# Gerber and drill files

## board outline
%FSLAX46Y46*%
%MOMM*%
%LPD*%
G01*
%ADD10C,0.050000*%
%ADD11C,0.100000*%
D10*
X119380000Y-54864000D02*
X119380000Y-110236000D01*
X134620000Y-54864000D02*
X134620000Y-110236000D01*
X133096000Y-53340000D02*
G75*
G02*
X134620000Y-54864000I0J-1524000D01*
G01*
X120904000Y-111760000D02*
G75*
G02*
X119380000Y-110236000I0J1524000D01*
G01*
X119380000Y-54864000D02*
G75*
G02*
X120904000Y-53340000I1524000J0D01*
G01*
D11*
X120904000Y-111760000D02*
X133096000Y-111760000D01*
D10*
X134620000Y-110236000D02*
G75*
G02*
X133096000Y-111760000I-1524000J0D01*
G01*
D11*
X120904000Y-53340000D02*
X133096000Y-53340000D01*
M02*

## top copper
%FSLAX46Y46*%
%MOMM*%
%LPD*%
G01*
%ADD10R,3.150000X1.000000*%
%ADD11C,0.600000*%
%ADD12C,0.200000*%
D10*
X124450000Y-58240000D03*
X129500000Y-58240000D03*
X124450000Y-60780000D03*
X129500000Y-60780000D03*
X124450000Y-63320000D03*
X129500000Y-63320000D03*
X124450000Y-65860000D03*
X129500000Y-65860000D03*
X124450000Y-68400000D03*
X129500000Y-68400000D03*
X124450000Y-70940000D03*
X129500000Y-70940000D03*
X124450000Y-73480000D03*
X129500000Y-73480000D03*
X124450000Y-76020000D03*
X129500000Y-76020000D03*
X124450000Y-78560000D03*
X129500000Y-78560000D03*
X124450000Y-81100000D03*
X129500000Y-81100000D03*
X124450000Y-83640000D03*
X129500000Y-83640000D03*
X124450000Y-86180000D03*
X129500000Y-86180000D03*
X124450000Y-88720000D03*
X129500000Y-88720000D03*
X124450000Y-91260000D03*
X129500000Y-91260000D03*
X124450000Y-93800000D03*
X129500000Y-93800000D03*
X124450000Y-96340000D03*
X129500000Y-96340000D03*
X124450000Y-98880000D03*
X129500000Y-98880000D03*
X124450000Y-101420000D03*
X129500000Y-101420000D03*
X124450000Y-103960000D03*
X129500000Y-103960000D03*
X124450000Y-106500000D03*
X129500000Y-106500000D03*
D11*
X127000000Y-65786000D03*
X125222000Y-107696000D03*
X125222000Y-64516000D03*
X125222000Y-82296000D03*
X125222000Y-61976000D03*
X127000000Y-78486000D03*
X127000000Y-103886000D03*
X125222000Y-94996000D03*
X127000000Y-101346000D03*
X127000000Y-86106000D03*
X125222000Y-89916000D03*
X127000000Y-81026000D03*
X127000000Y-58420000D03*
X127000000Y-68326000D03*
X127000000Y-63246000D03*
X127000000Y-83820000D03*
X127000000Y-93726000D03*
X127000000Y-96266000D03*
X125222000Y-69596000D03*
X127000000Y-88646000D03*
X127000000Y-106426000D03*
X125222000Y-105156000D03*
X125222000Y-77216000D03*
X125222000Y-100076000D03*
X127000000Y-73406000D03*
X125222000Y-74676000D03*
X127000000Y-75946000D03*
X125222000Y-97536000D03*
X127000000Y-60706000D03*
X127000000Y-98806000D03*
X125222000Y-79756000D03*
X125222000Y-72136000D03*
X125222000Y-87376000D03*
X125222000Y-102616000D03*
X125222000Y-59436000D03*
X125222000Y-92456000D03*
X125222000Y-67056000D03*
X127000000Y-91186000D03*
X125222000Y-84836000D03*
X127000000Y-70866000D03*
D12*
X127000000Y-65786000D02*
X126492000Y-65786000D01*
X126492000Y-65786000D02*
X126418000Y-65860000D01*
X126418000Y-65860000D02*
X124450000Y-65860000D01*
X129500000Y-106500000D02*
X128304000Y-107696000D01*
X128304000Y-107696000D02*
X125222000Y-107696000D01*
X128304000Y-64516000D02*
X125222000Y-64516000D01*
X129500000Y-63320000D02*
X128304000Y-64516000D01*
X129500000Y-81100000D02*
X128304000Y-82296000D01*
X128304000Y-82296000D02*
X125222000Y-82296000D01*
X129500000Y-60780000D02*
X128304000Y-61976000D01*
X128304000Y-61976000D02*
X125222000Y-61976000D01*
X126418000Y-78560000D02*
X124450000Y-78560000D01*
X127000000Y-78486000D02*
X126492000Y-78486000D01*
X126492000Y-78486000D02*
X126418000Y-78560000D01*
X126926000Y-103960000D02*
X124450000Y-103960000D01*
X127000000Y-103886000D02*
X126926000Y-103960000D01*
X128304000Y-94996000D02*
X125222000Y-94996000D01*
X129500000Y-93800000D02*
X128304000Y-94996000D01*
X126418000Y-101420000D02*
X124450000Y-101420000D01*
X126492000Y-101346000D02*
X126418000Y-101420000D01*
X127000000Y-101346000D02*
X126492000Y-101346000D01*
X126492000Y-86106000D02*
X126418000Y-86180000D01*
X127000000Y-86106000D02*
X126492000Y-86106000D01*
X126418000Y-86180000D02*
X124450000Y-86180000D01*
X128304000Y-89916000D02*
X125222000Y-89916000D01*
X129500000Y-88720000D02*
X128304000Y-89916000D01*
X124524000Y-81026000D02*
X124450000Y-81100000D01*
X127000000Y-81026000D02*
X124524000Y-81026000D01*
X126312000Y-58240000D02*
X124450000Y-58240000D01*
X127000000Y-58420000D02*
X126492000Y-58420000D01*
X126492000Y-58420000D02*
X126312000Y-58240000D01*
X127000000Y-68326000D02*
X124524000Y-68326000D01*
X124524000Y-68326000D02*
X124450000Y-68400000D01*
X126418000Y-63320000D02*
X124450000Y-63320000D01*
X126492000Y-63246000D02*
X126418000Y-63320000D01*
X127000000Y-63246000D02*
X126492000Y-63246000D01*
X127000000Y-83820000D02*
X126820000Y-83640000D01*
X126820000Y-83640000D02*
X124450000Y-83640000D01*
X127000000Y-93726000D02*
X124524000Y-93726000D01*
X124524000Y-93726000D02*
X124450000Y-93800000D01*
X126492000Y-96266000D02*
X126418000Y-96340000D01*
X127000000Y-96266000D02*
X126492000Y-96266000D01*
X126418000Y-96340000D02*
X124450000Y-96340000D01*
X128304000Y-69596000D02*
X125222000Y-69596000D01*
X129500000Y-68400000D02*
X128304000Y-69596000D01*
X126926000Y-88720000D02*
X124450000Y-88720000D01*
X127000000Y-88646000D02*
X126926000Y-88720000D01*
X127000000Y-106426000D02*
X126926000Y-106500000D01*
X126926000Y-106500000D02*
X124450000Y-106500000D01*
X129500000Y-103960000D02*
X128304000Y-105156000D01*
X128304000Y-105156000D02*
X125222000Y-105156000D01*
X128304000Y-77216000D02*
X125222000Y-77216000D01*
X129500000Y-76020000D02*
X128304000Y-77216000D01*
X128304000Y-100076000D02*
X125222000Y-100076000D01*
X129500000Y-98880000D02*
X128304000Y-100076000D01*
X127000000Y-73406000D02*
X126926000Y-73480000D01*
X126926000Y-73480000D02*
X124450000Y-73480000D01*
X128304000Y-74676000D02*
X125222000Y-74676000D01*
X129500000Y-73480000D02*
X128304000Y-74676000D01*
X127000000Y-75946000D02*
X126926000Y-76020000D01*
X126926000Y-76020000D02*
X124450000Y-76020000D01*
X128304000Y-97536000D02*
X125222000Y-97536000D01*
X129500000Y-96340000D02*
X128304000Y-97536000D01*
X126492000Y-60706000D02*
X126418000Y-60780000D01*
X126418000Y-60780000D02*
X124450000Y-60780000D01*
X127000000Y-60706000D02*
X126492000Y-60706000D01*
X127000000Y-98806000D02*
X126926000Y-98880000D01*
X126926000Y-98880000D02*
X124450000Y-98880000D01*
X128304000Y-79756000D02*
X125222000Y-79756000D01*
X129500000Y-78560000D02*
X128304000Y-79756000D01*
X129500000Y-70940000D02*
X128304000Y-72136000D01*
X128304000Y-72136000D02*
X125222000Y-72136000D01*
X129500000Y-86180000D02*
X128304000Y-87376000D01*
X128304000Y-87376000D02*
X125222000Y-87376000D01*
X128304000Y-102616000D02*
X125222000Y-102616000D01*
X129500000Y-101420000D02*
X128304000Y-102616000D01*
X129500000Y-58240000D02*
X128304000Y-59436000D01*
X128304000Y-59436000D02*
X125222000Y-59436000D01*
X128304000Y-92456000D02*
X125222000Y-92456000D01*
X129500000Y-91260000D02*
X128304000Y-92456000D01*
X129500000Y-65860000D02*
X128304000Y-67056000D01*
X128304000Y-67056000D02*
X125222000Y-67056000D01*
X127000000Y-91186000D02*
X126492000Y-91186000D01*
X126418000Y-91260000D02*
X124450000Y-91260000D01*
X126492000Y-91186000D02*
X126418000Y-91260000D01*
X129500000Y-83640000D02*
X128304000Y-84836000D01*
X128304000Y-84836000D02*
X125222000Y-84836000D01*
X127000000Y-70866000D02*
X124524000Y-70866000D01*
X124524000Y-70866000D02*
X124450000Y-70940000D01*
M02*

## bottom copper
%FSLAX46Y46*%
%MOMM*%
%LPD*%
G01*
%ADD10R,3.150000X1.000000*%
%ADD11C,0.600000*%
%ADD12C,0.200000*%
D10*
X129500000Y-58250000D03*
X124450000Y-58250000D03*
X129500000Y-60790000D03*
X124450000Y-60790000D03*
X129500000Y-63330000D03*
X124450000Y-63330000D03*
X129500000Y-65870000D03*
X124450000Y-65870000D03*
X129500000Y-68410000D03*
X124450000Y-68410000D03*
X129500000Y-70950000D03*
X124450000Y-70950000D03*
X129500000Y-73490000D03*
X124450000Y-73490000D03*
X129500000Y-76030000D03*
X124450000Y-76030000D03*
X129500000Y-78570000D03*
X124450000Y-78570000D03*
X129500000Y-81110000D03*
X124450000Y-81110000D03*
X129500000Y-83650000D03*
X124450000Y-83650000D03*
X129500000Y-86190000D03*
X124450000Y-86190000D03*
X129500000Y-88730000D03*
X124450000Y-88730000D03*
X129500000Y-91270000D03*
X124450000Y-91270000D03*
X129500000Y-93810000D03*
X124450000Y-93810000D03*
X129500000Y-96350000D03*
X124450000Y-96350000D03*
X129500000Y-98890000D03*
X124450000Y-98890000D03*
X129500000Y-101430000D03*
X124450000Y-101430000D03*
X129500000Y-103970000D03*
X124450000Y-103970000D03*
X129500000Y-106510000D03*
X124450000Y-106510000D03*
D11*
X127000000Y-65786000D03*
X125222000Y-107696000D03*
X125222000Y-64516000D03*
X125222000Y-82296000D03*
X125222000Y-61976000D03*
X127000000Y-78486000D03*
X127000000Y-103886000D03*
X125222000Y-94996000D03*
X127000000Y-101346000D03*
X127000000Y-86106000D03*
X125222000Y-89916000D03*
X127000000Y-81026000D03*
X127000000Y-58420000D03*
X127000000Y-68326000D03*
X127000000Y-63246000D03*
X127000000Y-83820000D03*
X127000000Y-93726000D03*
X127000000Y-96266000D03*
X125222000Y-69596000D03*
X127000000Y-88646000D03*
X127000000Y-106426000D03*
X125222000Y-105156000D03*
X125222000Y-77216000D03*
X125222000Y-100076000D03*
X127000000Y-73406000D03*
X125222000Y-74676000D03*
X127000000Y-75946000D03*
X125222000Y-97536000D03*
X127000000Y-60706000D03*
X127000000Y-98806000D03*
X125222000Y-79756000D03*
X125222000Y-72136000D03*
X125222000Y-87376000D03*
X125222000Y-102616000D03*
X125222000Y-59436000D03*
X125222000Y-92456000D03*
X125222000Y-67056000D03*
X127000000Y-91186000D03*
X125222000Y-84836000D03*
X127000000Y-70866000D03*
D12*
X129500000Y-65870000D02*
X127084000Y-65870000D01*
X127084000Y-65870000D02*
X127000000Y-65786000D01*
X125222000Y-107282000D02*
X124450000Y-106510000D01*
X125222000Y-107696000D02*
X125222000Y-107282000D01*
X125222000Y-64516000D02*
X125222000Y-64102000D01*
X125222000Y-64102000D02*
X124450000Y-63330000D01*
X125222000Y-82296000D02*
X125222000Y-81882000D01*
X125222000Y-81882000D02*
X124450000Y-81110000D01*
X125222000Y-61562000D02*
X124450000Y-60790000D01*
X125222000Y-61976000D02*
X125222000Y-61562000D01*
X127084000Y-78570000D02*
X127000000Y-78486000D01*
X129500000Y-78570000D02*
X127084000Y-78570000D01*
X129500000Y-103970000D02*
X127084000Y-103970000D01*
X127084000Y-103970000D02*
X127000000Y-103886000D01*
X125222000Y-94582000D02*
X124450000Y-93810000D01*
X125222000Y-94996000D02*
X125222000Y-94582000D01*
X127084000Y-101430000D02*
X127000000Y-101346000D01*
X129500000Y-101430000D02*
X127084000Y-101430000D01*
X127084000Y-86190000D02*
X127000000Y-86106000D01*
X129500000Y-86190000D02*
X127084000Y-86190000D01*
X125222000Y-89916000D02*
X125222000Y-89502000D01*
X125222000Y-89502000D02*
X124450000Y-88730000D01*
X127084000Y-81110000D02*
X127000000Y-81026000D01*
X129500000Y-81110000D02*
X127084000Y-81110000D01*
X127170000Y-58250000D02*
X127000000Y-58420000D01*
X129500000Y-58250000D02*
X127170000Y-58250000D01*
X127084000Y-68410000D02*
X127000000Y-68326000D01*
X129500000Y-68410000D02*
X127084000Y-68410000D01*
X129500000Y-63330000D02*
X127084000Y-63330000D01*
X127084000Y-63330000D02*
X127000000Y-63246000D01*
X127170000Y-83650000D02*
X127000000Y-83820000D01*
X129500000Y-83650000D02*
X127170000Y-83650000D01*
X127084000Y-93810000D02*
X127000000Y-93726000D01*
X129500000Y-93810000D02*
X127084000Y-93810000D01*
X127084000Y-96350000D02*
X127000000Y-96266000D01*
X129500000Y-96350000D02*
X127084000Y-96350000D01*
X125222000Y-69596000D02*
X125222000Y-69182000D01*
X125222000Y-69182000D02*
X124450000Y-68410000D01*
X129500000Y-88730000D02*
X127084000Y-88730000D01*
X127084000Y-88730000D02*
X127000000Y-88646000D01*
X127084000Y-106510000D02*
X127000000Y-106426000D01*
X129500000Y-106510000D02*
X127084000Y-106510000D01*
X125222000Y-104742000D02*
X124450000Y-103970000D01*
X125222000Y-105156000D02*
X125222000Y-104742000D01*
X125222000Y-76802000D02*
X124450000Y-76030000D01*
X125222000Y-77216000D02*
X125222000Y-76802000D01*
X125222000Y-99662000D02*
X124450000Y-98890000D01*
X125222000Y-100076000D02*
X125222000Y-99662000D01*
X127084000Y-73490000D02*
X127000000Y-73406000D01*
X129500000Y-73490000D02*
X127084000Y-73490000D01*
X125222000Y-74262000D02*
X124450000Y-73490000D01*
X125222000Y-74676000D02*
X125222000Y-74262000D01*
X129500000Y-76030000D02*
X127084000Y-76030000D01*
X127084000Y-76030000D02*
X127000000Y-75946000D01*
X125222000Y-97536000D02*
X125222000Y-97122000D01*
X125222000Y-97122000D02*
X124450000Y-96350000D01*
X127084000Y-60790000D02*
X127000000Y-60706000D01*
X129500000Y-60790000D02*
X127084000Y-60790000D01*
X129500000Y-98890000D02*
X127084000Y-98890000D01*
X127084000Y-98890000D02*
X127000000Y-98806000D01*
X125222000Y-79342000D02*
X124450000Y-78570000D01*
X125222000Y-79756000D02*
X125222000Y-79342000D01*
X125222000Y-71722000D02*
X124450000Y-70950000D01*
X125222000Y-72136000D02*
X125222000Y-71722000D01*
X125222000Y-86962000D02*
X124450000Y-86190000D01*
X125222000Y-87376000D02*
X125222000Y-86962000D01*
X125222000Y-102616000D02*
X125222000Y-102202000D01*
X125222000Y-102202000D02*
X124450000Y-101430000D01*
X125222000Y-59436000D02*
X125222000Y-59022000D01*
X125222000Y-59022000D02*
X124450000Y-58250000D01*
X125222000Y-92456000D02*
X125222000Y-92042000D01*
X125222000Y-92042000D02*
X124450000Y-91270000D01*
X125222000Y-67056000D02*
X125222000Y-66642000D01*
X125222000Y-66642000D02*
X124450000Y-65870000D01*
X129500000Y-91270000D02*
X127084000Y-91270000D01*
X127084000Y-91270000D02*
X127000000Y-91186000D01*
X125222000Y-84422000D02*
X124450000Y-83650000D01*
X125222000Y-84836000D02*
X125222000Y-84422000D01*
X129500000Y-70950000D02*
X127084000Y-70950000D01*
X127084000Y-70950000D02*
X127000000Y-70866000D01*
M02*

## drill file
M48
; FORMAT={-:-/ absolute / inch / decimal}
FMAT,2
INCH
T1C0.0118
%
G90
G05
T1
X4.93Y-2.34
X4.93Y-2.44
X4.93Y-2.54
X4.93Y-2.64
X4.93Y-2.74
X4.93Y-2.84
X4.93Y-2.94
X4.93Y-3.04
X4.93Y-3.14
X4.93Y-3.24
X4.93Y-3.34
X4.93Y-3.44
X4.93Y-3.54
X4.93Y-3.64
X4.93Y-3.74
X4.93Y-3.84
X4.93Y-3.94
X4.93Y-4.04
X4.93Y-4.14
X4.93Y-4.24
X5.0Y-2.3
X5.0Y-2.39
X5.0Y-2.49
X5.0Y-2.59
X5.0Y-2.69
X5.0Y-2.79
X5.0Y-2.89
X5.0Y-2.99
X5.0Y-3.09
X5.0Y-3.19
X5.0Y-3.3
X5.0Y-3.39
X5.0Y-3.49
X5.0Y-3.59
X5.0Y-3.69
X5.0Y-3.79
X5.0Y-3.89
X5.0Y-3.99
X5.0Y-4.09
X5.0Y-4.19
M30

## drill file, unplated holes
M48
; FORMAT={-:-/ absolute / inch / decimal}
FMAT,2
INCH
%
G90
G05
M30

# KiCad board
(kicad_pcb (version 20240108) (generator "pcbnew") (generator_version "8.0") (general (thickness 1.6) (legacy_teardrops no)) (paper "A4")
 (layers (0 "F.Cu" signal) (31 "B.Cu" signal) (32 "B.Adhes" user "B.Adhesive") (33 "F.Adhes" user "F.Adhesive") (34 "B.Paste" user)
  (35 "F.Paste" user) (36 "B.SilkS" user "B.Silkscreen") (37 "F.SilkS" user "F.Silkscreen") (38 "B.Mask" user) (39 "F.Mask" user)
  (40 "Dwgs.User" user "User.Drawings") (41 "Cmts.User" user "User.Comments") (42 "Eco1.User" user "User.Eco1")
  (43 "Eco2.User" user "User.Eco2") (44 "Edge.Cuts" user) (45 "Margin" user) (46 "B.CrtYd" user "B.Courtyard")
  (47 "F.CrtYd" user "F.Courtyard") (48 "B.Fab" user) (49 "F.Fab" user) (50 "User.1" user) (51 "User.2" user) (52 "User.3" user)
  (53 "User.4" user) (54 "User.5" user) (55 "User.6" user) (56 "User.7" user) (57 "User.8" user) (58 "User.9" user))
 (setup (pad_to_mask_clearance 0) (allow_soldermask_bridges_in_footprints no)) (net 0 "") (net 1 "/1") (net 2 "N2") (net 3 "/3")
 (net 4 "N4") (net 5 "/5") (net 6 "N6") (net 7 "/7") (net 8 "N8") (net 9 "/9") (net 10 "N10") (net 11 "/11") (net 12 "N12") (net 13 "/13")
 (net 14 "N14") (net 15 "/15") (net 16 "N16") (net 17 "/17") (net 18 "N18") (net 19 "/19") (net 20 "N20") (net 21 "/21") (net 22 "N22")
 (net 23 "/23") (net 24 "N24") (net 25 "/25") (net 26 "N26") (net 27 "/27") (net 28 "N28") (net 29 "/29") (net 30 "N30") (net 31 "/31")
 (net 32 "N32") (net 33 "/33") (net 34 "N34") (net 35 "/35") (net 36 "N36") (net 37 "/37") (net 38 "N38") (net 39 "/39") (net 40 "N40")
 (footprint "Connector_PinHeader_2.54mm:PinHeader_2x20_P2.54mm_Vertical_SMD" (layer "F.Cu") (at 126.975 82.37)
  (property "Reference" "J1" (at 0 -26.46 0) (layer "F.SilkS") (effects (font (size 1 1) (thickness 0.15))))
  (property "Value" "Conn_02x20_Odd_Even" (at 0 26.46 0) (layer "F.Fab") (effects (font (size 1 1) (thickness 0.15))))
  (pad "1" smd rect (at -2.525 -24.13) (size 3.15 1) (layers "F.Cu" "F.Paste" "F.Mask") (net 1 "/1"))
  (pad "2" smd rect (at 2.525 -24.13) (size 3.15 1) (layers "F.Cu" "F.Paste" "F.Mask") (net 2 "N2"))
  (pad "3" smd rect (at -2.525 -21.59) (size 3.15 1) (layers "F.Cu" "F.Paste" "F.Mask") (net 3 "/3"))
  (pad "4" smd rect (at 2.525 -21.59) (size 3.15 1) (layers "F.Cu" "F.Paste" "F.Mask") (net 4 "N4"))
  (pad "5" smd rect (at -2.525 -19.05) (size 3.15 1) (layers "F.Cu" "F.Paste" "F.Mask") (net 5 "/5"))
  (pad "6" smd rect (at 2.525 -19.05) (size 3.15 1) (layers "F.Cu" "F.Paste" "F.Mask") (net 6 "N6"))
  (pad "7" smd rect (at -2.525 -16.51) (size 3.15 1) (layers "F.Cu" "F.Paste" "F.Mask") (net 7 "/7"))
  (pad "8" smd rect (at 2.525 -16.51) (size 3.15 1) (layers "F.Cu" "F.Paste" "F.Mask") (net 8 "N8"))
  (pad "9" smd rect (at -2.525 -13.97) (size 3.15 1) (layers "F.Cu" "F.Paste" "F.Mask") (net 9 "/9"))
  (pad "10" smd rect (at 2.525 -13.97) (size 3.15 1) (layers "F.Cu" "F.Paste" "F.Mask") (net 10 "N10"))
  (pad "11" smd rect (at -2.525 -11.43) (size 3.15 1) (layers "F.Cu" "F.Paste" "F.Mask") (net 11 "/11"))
  (pad "12" smd rect (at 2.525 -11.43) (size 3.15 1) (layers "F.Cu" "F.Paste" "F.Mask") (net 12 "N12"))
  (pad "13" smd rect (at -2.525 -8.89) (size 3.15 1) (layers "F.Cu" "F.Paste" "F.Mask") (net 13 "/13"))
  (pad "14" smd rect (at 2.525 -8.89) (size 3.15 1) (layers "F.Cu" "F.Paste" "F.Mask") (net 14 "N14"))
  (pad "15" smd rect (at -2.525 -6.35) (size 3.15 1) (layers "F.Cu" "F.Paste" "F.Mask") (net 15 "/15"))
  (pad "16" smd rect (at 2.525 -6.35) (size 3.15 1) (layers "F.Cu" "F.Paste" "F.Mask") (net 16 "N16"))
  (pad "17" smd rect (at -2.525 -3.81) (size 3.15 1) (layers "F.Cu" "F.Paste" "F.Mask") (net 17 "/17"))
  (pad "18" smd rect (at 2.525 -3.81) (size 3.15 1) (layers "F.Cu" "F.Paste" "F.Mask") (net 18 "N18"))
  (pad "19" smd rect (at -2.525 -1.27) (size 3.15 1) (layers "F.Cu" "F.Paste" "F.Mask") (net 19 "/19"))
  (pad "20" smd rect (at 2.525 -1.27) (size 3.15 1) (layers "F.Cu" "F.Paste" "F.Mask") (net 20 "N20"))
  (pad "21" smd rect (at -2.525 1.27) (size 3.15 1) (layers "F.Cu" "F.Paste" "F.Mask") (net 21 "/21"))
  (pad "22" smd rect (at 2.525 1.27) (size 3.15 1) (layers "F.Cu" "F.Paste" "F.Mask") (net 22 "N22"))
  (pad "23" smd rect (at -2.525 3.81) (size 3.15 1) (layers "F.Cu" "F.Paste" "F.Mask") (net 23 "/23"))
  (pad "24" smd rect (at 2.525 3.81) (size 3.15 1) (layers "F.Cu" "F.Paste" "F.Mask") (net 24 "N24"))
  (pad "25" smd rect (at -2.525 6.35) (size 3.15 1) (layers "F.Cu" "F.Paste" "F.Mask") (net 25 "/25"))
  (pad "26" smd rect (at 2.525 6.35) (size 3.15 1) (layers "F.Cu" "F.Paste" "F.Mask") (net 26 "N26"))
  (pad "27" smd rect (at -2.525 8.89) (size 3.15 1) (layers "F.Cu" "F.Paste" "F.Mask") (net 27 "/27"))
  (pad "28" smd rect (at 2.525 8.89) (size 3.15 1) (layers "F.Cu" "F.Paste" "F.Mask") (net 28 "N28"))
  (pad "29" smd rect (at -2.525 11.43) (size 3.15 1) (layers "F.Cu" "F.Paste" "F.Mask") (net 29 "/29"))
  (pad "30" smd rect (at 2.525 11.43) (size 3.15 1) (layers "F.Cu" "F.Paste" "F.Mask") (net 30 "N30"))
  (pad "31" smd rect (at -2.525 13.97) (size 3.15 1) (layers "F.Cu" "F.Paste" "F.Mask") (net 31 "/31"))
  (pad "32" smd rect (at 2.525 13.97) (size 3.15 1) (layers "F.Cu" "F.Paste" "F.Mask") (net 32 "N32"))
  (pad "33" smd rect (at -2.525 16.51) (size 3.15 1) (layers "F.Cu" "F.Paste" "F.Mask") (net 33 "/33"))
  (pad "34" smd rect (at 2.525 16.51) (size 3.15 1) (layers "F.Cu" "F.Paste" "F.Mask") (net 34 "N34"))
  (pad "35" smd rect (at -2.525 19.05) (size 3.15 1) (layers "F.Cu" "F.Paste" "F.Mask") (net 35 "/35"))
  (pad "36" smd rect (at 2.525 19.05) (size 3.15 1) (layers "F.Cu" "F.Paste" "F.Mask") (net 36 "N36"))
  (pad "37" smd rect (at -2.525 21.59) (size 3.15 1) (layers "F.Cu" "F.Paste" "F.Mask") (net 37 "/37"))
  (pad "38" smd rect (at 2.525 21.59) (size 3.15 1) (layers "F.Cu" "F.Paste" "F.Mask") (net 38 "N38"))
  (pad "39" smd rect (at -2.525 24.13) (size 3.15 1) (layers "F.Cu" "F.Paste" "F.Mask") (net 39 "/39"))
  (pad "40" smd rect (at 2.525 24.13) (size 3.15 1) (layers "F.Cu" "F.Paste" "F.Mask") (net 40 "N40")))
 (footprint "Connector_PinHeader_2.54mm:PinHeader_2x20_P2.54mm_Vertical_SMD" (layer "B.Cu") (at 126.975 82.38 180)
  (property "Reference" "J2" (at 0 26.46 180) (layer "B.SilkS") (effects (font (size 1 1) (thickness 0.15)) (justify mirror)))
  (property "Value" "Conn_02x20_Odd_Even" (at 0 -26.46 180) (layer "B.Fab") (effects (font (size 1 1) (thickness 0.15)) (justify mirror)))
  (pad "1" smd rect (at -2.525 24.13 180) (size 3.15 1) (layers "B.Cu" "B.Paste" "B.Mask") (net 1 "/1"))
  (pad "2" smd rect (at 2.525 24.13 180) (size 3.15 1) (layers "B.Cu" "B.Paste" "B.Mask") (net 2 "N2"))
  (pad "3" smd rect (at -2.525 21.59 180) (size 3.15 1) (layers "B.Cu" "B.Paste" "B.Mask") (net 3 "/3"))
  (pad "4" smd rect (at 2.525 21.59 180) (size 3.15 1) (layers "B.Cu" "B.Paste" "B.Mask") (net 4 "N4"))
  (pad "5" smd rect (at -2.525 19.05 180) (size 3.15 1) (layers "B.Cu" "B.Paste" "B.Mask") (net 5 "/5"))
  (pad "6" smd rect (at 2.525 19.05 180) (size 3.15 1) (layers "B.Cu" "B.Paste" "B.Mask") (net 6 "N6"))
  (pad "7" smd rect (at -2.525 16.51 180) (size 3.15 1) (layers "B.Cu" "B.Paste" "B.Mask") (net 7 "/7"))
  (pad "8" smd rect (at 2.525 16.51 180) (size 3.15 1) (layers "B.Cu" "B.Paste" "B.Mask") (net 8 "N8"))
  (pad "9" smd rect (at -2.525 13.97 180) (size 3.15 1) (layers "B.Cu" "B.Paste" "B.Mask") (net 9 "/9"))
  (pad "10" smd rect (at 2.525 13.97 180) (size 3.15 1) (layers "B.Cu" "B.Paste" "B.Mask") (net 10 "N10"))
  (pad "11" smd rect (at -2.525 11.43 180) (size 3.15 1) (layers "B.Cu" "B.Paste" "B.Mask") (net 11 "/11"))
  (pad "12" smd rect (at 2.525 11.43 180) (size 3.15 1) (layers "B.Cu" "B.Paste" "B.Mask") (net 12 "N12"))
  (pad "13" smd rect (at -2.525 8.89 180) (size 3.15 1) (layers "B.Cu" "B.Paste" "B.Mask") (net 13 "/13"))
  (pad "14" smd rect (at 2.525 8.89 180) (size 3.15 1) (layers "B.Cu" "B.Paste" "B.Mask") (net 14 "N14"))
  (pad "15" smd rect (at -2.525 6.35 180) (size 3.15 1) (layers "B.Cu" "B.Paste" "B.Mask") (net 15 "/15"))
  (pad "16" smd rect (at 2.525 6.35 180) (size 3.15 1) (layers "B.Cu" "B.Paste" "B.Mask") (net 16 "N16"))
  (pad "17" smd rect (at -2.525 3.81 180) (size 3.15 1) (layers "B.Cu" "B.Paste" "B.Mask") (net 17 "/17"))
  (pad "18" smd rect (at 2.525 3.81 180) (size 3.15 1) (layers "B.Cu" "B.Paste" "B.Mask") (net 18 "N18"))
  (pad "19" smd rect (at -2.525 1.27 180) (size 3.15 1) (layers "B.Cu" "B.Paste" "B.Mask") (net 19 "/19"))
  (pad "20" smd rect (at 2.525 1.27 180) (size 3.15 1) (layers "B.Cu" "B.Paste" "B.Mask") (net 20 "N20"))
  (pad "21" smd rect (at -2.525 -1.27 180) (size 3.15 1) (layers "B.Cu" "B.Paste" "B.Mask") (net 21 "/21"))
  (pad "22" smd rect (at 2.525 -1.27 180) (size 3.15 1) (layers "B.Cu" "B.Paste" "B.Mask") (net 22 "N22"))
  (pad "23" smd rect (at -2.525 -3.81 180) (size 3.15 1) (layers "B.Cu" "B.Paste" "B.Mask") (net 23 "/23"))
  (pad "24" smd rect (at 2.525 -3.81 180) (size 3.15 1) (layers "B.Cu" "B.Paste" "B.Mask") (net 24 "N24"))
  (pad "25" smd rect (at -2.525 -6.35 180) (size 3.15 1) (layers "B.Cu" "B.Paste" "B.Mask") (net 25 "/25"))
  (pad "26" smd rect (at 2.525 -6.35 180) (size 3.15 1) (layers "B.Cu" "B.Paste" "B.Mask") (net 26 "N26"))
  (pad "27" smd rect (at -2.525 -8.89 180) (size 3.15 1) (layers "B.Cu" "B.Paste" "B.Mask") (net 27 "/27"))
  (pad "28" smd rect (at 2.525 -8.89 180) (size 3.15 1) (layers "B.Cu" "B.Paste" "B.Mask") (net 28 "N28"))
  (pad "29" smd rect (at -2.525 -11.43 180) (size 3.15 1) (layers "B.Cu" "B.Paste" "B.Mask") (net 29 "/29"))
  (pad "30" smd rect (at 2.525 -11.43 180) (size 3.15 1) (layers "B.Cu" "B.Paste" "B.Mask") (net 30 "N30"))
  (pad "31" smd rect (at -2.525 -13.97 180) (size 3.15 1) (layers "B.Cu" "B.Paste" "B.Mask") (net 31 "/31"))
  (pad "32" smd rect (at 2.525 -13.97 180) (size 3.15 1) (layers "B.Cu" "B.Paste" "B.Mask") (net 32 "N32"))
  (pad "33" smd rect (at -2.525 -16.51 180) (size 3.15 1) (layers "B.Cu" "B.Paste" "B.Mask") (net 33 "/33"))
  (pad "34" smd rect (at 2.525 -16.51 180) (size 3.15 1) (layers "B.Cu" "B.Paste" "B.Mask") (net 34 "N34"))
  (pad "35" smd rect (at -2.525 -19.05 180) (size 3.15 1) (layers "B.Cu" "B.Paste" "B.Mask") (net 35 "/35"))
  (pad "36" smd rect (at 2.525 -19.05 180) (size 3.15 1) (layers "B.Cu" "B.Paste" "B.Mask") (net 36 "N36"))
  (pad "37" smd rect (at -2.525 -21.59 180) (size 3.15 1) (layers "B.Cu" "B.Paste" "B.Mask") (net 37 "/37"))
  (pad "38" smd rect (at 2.525 -21.59 180) (size 3.15 1) (layers "B.Cu" "B.Paste" "B.Mask") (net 38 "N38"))
  (pad "39" smd rect (at -2.525 -24.13 180) (size 3.15 1) (layers "B.Cu" "B.Paste" "B.Mask") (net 39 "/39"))
  (pad "40" smd rect (at 2.525 -24.13 180) (size 3.15 1) (layers "B.Cu" "B.Paste" "B.Mask") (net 40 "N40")))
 (gr_line (start 119.38 54.864) (end 119.38 110.236) (stroke (width 0.05) (type default)) (layer "Edge.Cuts"))
 (gr_line (start 134.62 54.864) (end 134.62 110.236) (stroke (width 0.05) (type default)) (layer "Edge.Cuts"))
 (gr_arc (start 133.096 53.34) (mid 134.173631 53.786369) (end 134.62 54.864) (stroke (width 0.05) (type default)) (layer "Edge.Cuts"))
 (gr_arc (start 120.904 111.76) (mid 119.826369 111.313631) (end 119.38 110.236) (stroke (width 0.05) (type default)) (layer "Edge.Cuts"))
 (gr_arc (start 119.38 54.864) (mid 119.826369 53.786369) (end 120.904 53.34) (stroke (width 0.05) (type default)) (layer "Edge.Cuts"))
 (gr_line (start 120.904 111.76) (end 133.096 111.76) (stroke (width 0.1) (type default)) (layer "Edge.Cuts"))
 (gr_arc (start 134.62 110.236) (mid 134.173631 111.313631) (end 133.096 111.76) (stroke (width 0.05) (type default)) (layer "Edge.Cuts"))
 (gr_line (start 120.904 53.34) (end 133.096 53.34) (stroke (width 0.1) (type default)) (layer "Edge.Cuts"))
 (segment (start 127 65.786) (end 126.492 65.786) (width 0.2) (layer "F.Cu") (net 7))
 (segment (start 126.492 65.786) (end 126.418 65.86) (width 0.2) (layer "F.Cu") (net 7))
 (segment (start 126.418 65.86) (end 124.45 65.86) (width 0.2) (layer "F.Cu") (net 7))
 (via (at 127 65.786) (size 0.6) (drill 0.3) (layers "F.Cu" "B.Cu") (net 7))
 (segment (start 129.5 65.87) (end 127.084 65.87) (width 0.2) (layer "B.Cu") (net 7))
 (segment (start 127.084 65.87) (end 127 65.786) (width 0.2) (layer "B.Cu") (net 7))
 (segment (start 129.5 106.5) (end 128.304 107.696) (width 0.2) (layer "F.Cu") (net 40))
 (segment (start 128.304 107.696) (end 125.222 107.696) (width 0.2) (layer "F.Cu") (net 40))
 (via (at 125.222 107.696) (size 0.6) (drill 0.3) (layers "F.Cu" "B.Cu") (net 40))
 (segment (start 125.222 107.282) (end 124.45 106.51) (width 0.2) (layer "B.Cu") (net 40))
 (segment (start 125.222 107.696) (end 125.222 107.282) (width 0.2) (layer "B.Cu") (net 40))
 (segment (start 128.304 64.516) (end 125.222 64.516) (width 0.2) (layer "F.Cu") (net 6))
 (segment (start 129.5 63.32) (end 128.304 64.516) (width 0.2) (layer "F.Cu") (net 6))
 (via (at 125.222 64.516) (size 0.6) (drill 0.3) (layers "F.Cu" "B.Cu") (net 6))
 (segment (start 125.222 64.516) (end 125.222 64.102) (width 0.2) (layer "B.Cu") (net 6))
 (segment (start 125.222 64.102) (end 124.45 63.33) (width 0.2) (layer "B.Cu") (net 6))
 (segment (start 129.5 81.1) (end 128.304 82.296) (width 0.2) (layer "F.Cu") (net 20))
 (segment (start 128.304 82.296) (end 125.222 82.296) (width 0.2) (layer "F.Cu") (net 20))
 (via (at 125.222 82.296) (size 0.6) (drill 0.3) (layers "F.Cu" "B.Cu") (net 20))
 (segment (start 125.222 82.296) (end 125.222 81.882) (width 0.2) (layer "B.Cu") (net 20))
 (segment (start 125.222 81.882) (end 124.45 81.11) (width 0.2) (layer "B.Cu") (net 20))
 (segment (start 129.5 60.78) (end 128.304 61.976) (width 0.2) (layer "F.Cu") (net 4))
 (segment (start 128.304 61.976) (end 125.222 61.976) (width 0.2) (layer "F.Cu") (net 4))
 (via (at 125.222 61.976) (size 0.6) (drill 0.3) (layers "F.Cu" "B.Cu") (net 4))
 (segment (start 125.222 61.562) (end 124.45 60.79) (width 0.2) (layer "B.Cu") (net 4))
 (segment (start 125.222 61.976) (end 125.222 61.562) (width 0.2) (layer "B.Cu") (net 4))
 (segment (start 126.418 78.56) (end 124.45 78.56) (width 0.2) (layer "F.Cu") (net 17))
 (segment (start 127 78.486) (end 126.492 78.486) (width 0.2) (layer "F.Cu") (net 17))
 (segment (start 126.492 78.486) (end 126.418 78.56) (width 0.2) (layer "F.Cu") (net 17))
 (via (at 127 78.486) (size 0.6) (drill 0.3) (layers "F.Cu" "B.Cu") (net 17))
 (segment (start 127.084 78.57) (end 127 78.486) (width 0.2) (layer "B.Cu") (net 17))
 (segment (start 129.5 78.57) (end 127.084 78.57) (width 0.2) (layer "B.Cu") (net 17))
 (segment (start 126.926 103.96) (end 124.45 103.96) (width 0.2) (layer "F.Cu") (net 37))
 (segment (start 127 103.886) (end 126.926 103.96) (width 0.2) (layer "F.Cu") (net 37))
 (via (at 127 103.886) (size 0.6) (drill 0.3) (layers "F.Cu" "B.Cu") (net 37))
 (segment (start 129.5 103.97) (end 127.084 103.97) (width 0.2) (layer "B.Cu") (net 37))
 (segment (start 127.084 103.97) (end 127 103.886) (width 0.2) (layer "B.Cu") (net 37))
 (segment (start 128.304 94.996) (end 125.222 94.996) (width 0.2) (layer "F.Cu") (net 30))
 (segment (start 129.5 93.8) (end 128.304 94.996) (width 0.2) (layer "F.Cu") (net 30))
 (via (at 125.222 94.996) (size 0.6) (drill 0.3) (layers "F.Cu" "B.Cu") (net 30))
 (segment (start 125.222 94.582) (end 124.45 93.81) (width 0.2) (layer "B.Cu") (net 30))
 (segment (start 125.222 94.996) (end 125.222 94.582) (width 0.2) (layer "B.Cu") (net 30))
 (segment (start 126.418 101.42) (end 124.45 101.42) (width 0.2) (layer "F.Cu") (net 35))
 (segment (start 126.492 101.346) (end 126.418 101.42) (width 0.2) (layer "F.Cu") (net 35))
 (segment (start 127 101.346) (end 126.492 101.346) (width 0.2) (layer "F.Cu") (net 35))
 (via (at 127 101.346) (size 0.6) (drill 0.3) (layers "F.Cu" "B.Cu") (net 35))
 (segment (start 127.084 101.43) (end 127 101.346) (width 0.2) (layer "B.Cu") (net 35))
 (segment (start 129.5 101.43) (end 127.084 101.43) (width 0.2) (layer "B.Cu") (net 35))
 (segment (start 126.492 86.106) (end 126.418 86.18) (width 0.2) (layer "F.Cu") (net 23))
 (segment (start 127 86.106) (end 126.492 86.106) (width 0.2) (layer "F.Cu") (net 23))
 (segment (start 126.418 86.18) (end 124.45 86.18) (width 0.2) (layer "F.Cu") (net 23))
 (via (at 127 86.106) (size 0.6) (drill 0.3) (layers "F.Cu" "B.Cu") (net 23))
 (segment (start 127.084 86.19) (end 127 86.106) (width 0.2) (layer "B.Cu") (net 23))
 (segment (start 129.5 86.19) (end 127.084 86.19) (width 0.2) (layer "B.Cu") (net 23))
 (segment (start 128.304 89.916) (end 125.222 89.916) (width 0.2) (layer "F.Cu") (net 26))
 (segment (start 129.5 88.72) (end 128.304 89.916) (width 0.2) (layer "F.Cu") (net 26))
 (via (at 125.222 89.916) (size 0.6) (drill 0.3) (layers "F.Cu" "B.Cu") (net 26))
 (segment (start 125.222 89.916) (end 125.222 89.502) (width 0.2) (layer "B.Cu") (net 26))
 (segment (start 125.222 89.502) (end 124.45 88.73) (width 0.2) (layer "B.Cu") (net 26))
 (segment (start 124.524 81.026) (end 124.45 81.1) (width 0.2) (layer "F.Cu") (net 19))
 (segment (start 127 81.026) (end 124.524 81.026) (width 0.2) (layer "F.Cu") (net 19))
 (via (at 127 81.026) (size 0.6) (drill 0.3) (layers "F.Cu" "B.Cu") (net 19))
 (segment (start 127.084 81.11) (end 127 81.026) (width 0.2) (layer "B.Cu") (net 19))
 (segment (start 129.5 81.11) (end 127.084 81.11) (width 0.2) (layer "B.Cu") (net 19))
 (segment (start 126.312 58.24) (end 124.45 58.24) (width 0.2) (layer "F.Cu") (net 1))
 (segment (start 127 58.42) (end 126.492 58.42) (width 0.2) (layer "F.Cu") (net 1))
 (segment (start 126.492 58.42) (end 126.312 58.24) (width 0.2) (layer "F.Cu") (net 1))
 (via (at 127 58.42) (size 0.6) (drill 0.3) (layers "F.Cu" "B.Cu") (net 1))
 (segment (start 127.17 58.25) (end 127 58.42) (width 0.2) (layer "B.Cu") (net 1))
 (segment (start 129.5 58.25) (end 127.17 58.25) (width 0.2) (layer "B.Cu") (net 1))
 (segment (start 127 68.326) (end 124.524 68.326) (width 0.2) (layer "F.Cu") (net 9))
 (segment (start 124.524 68.326) (end 124.45 68.4) (width 0.2) (layer "F.Cu") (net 9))
 (via (at 127 68.326) (size 0.6) (drill 0.3) (layers "F.Cu" "B.Cu") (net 9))
 (segment (start 127.084 68.41) (end 127 68.326) (width 0.2) (layer "B.Cu") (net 9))
 (segment (start 129.5 68.41) (end 127.084 68.41) (width 0.2) (layer "B.Cu") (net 9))
 (segment (start 126.418 63.32) (end 124.45 63.32) (width 0.2) (layer "F.Cu") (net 5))
 (segment (start 126.492 63.246) (end 126.418 63.32) (width 0.2) (layer "F.Cu") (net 5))
 (segment (start 127 63.246) (end 126.492 63.246) (width 0.2) (layer "F.Cu") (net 5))
 (via (at 127 63.246) (size 0.6) (drill 0.3) (layers "F.Cu" "B.Cu") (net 5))
 (segment (start 129.5 63.33) (end 127.084 63.33) (width 0.2) (layer "B.Cu") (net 5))
 (segment (start 127.084 63.33) (end 127 63.246) (width 0.2) (layer "B.Cu") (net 5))
 (segment (start 127 83.82) (end 126.82 83.64) (width 0.2) (layer "F.Cu") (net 21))
 (segment (start 126.82 83.64) (end 124.45 83.64) (width 0.2) (layer "F.Cu") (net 21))
 (via (at 127 83.82) (size 0.6) (drill 0.3) (layers "F.Cu" "B.Cu") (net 21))
 (segment (start 127.17 83.65) (end 127 83.82) (width 0.2) (layer "B.Cu") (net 21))
 (segment (start 129.5 83.65) (end 127.17 83.65) (width 0.2) (layer "B.Cu") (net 21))
 (segment (start 127 93.726) (end 124.524 93.726) (width 0.2) (layer "F.Cu") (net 29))
 (segment (start 124.524 93.726) (end 124.45 93.8) (width 0.2) (layer "F.Cu") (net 29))
 (via (at 127 93.726) (size 0.6) (drill 0.3) (layers "F.Cu" "B.Cu") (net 29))
 (segment (start 127.084 93.81) (end 127 93.726) (width 0.2) (layer "B.Cu") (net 29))
 (segment (start 129.5 93.81) (end 127.084 93.81) (width 0.2) (layer "B.Cu") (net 29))
 (segment (start 126.492 96.266) (end 126.418 96.34) (width 0.2) (layer "F.Cu") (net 31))
 (segment (start 127 96.266) (end 126.492 96.266) (width 0.2) (layer "F.Cu") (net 31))
 (segment (start 126.418 96.34) (end 124.45 96.34) (width 0.2) (layer "F.Cu") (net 31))
 (via (at 127 96.266) (size 0.6) (drill 0.3) (layers "F.Cu" "B.Cu") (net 31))
 (segment (start 127.084 96.35) (end 127 96.266) (width 0.2) (layer "B.Cu") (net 31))
 (segment (start 129.5 96.35) (end 127.084 96.35) (width 0.2) (layer "B.Cu") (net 31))
 (segment (start 128.304 69.596) (end 125.222 69.596) (width 0.2) (layer "F.Cu") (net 10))
 (segment (start 129.5 68.4) (end 128.304 69.596) (width 0.2) (layer "F.Cu") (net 10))
 (via (at 125.222 69.596) (size 0.6) (drill 0.3) (layers "F.Cu" "B.Cu") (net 10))
 (segment (start 125.222 69.596) (end 125.222 69.182) (width 0.2) (layer "B.Cu") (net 10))
 (segment (start 125.222 69.182) (end 124.45 68.41) (width 0.2) (layer "B.Cu") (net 10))
 (segment (start 126.926 88.72) (end 124.45 88.72) (width 0.2) (layer "F.Cu") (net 25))
 (segment (start 127 88.646) (end 126.926 88.72) (width 0.2) (layer "F.Cu") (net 25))
 (via (at 127 88.646) (size 0.6) (drill 0.3) (layers "F.Cu" "B.Cu") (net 25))
 (segment (start 129.5 88.73) (end 127.084 88.73) (width 0.2) (layer "B.Cu") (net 25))
 (segment (start 127.084 88.73) (end 127 88.646) (width 0.2) (layer "B.Cu") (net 25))
 (segment (start 127 106.426) (end 126.926 106.5) (width 0.2) (layer "F.Cu") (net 39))
 (segment (start 126.926 106.5) (end 124.45 106.5) (width 0.2) (layer "F.Cu") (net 39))
 (via (at 127 106.426) (size 0.6) (drill 0.3) (layers "F.Cu" "B.Cu") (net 39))
 (segment (start 127.084 106.51) (end 127 106.426) (width 0.2) (layer "B.Cu") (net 39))
 (segment (start 129.5 106.51) (end 127.084 106.51) (width 0.2) (layer "B.Cu") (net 39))
 (segment (start 129.5 103.96) (end 128.304 105.156) (width 0.2) (layer "F.Cu") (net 38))
 (segment (start 128.304 105.156) (end 125.222 105.156) (width 0.2) (layer "F.Cu") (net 38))
 (via (at 125.222 105.156) (size 0.6) (drill 0.3) (layers "F.Cu" "B.Cu") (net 38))
 (segment (start 125.222 104.742) (end 124.45 103.97) (width 0.2) (layer "B.Cu") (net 38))
 (segment (start 125.222 105.156) (end 125.222 104.742) (width 0.2) (layer "B.Cu") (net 38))
 (segment (start 128.304 77.216) (end 125.222 77.216) (width 0.2) (layer "F.Cu") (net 16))
 (segment (start 129.5 76.02) (end 128.304 77.216) (width 0.2) (layer "F.Cu") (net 16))
 (via (at 125.222 77.216) (size 0.6) (drill 0.3) (layers "F.Cu" "B.Cu") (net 16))
 (segment (start 125.222 76.802) (end 124.45 76.03) (width 0.2) (layer "B.Cu") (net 16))
 (segment (start 125.222 77.216) (end 125.222 76.802) (width 0.2) (layer "B.Cu") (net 16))
 (segment (start 128.304 100.076) (end 125.222 100.076) (width 0.2) (layer "F.Cu") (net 34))
 (segment (start 129.5 98.88) (end 128.304 100.076) (width 0.2) (layer "F.Cu") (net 34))
 (via (at 125.222 100.076) (size 0.6) (drill 0.3) (layers "F.Cu" "B.Cu") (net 34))
 (segment (start 125.222 99.662) (end 124.45 98.89) (width 0.2) (layer "B.Cu") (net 34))
 (segment (start 125.222 100.076) (end 125.222 99.662) (width 0.2) (layer "B.Cu") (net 34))
 (segment (start 127 73.406) (end 126.926 73.48) (width 0.2) (layer "F.Cu") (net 13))
 (segment (start 126.926 73.48) (end 124.45 73.48) (width 0.2) (layer "F.Cu") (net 13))
 (via (at 127 73.406) (size 0.6) (drill 0.3) (layers "F.Cu" "B.Cu") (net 13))
 (segment (start 127.084 73.49) (end 127 73.406) (width 0.2) (layer "B.Cu") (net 13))
 (segment (start 129.5 73.49) (end 127.084 73.49) (width 0.2) (layer "B.Cu") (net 13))
 (segment (start 128.304 74.676) (end 125.222 74.676) (width 0.2) (layer "F.Cu") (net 14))
 (segment (start 129.5 73.48) (end 128.304 74.676) (width 0.2) (layer "F.Cu") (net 14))
 (via (at 125.222 74.676) (size 0.6) (drill 0.3) (layers "F.Cu" "B.Cu") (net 14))
 (segment (start 125.222 74.262) (end 124.45 73.49) (width 0.2) (layer "B.Cu") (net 14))
 (segment (start 125.222 74.676) (end 125.222 74.262) (width 0.2) (layer "B.Cu") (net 14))
 (segment (start 127 75.946) (end 126.926 76.02) (width 0.2) (layer "F.Cu") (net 15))
 (segment (start 126.926 76.02) (end 124.45 76.02) (width 0.2) (layer "F.Cu") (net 15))
 (via (at 127 75.946) (size 0.6) (drill 0.3) (layers "F.Cu" "B.Cu") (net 15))
 (segment (start 129.5 76.03) (end 127.084 76.03) (width 0.2) (layer "B.Cu") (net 15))
 (segment (start 127.084 76.03) (end 127 75.946) (width 0.2) (layer "B.Cu") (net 15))
 (segment (start 128.304 97.536) (end 125.222 97.536) (width 0.2) (layer "F.Cu") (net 32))
 (segment (start 129.5 96.34) (end 128.304 97.536) (width 0.2) (layer "F.Cu") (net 32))
 (via (at 125.222 97.536) (size 0.6) (drill 0.3) (layers "F.Cu" "B.Cu") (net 32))
 (segment (start 125.222 97.536) (end 125.222 97.122) (width 0.2) (layer "B.Cu") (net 32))
 (segment (start 125.222 97.122) (end 124.45 96.35) (width 0.2) (layer "B.Cu") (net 32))
 (segment (start 126.492 60.706) (end 126.418 60.78) (width 0.2) (layer "F.Cu") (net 3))
 (segment (start 126.418 60.78) (end 124.45 60.78) (width 0.2) (layer "F.Cu") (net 3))
 (segment (start 127 60.706) (end 126.492 60.706) (width 0.2) (layer "F.Cu") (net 3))
 (via (at 127 60.706) (size 0.6) (drill 0.3) (layers "F.Cu" "B.Cu") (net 3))
 (segment (start 127.084 60.79) (end 127 60.706) (width 0.2) (layer "B.Cu") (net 3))
 (segment (start 129.5 60.79) (end 127.084 60.79) (width 0.2) (layer "B.Cu") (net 3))
 (segment (start 127 98.806) (end 126.926 98.88) (width 0.2) (layer "F.Cu") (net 33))
 (segment (start 126.926 98.88) (end 124.45 98.88) (width 0.2) (layer "F.Cu") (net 33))
 (via (at 127 98.806) (size 0.6) (drill 0.3) (layers "F.Cu" "B.Cu") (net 33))
 (segment (start 129.5 98.89) (end 127.084 98.89) (width 0.2) (layer "B.Cu") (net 33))
 (segment (start 127.084 98.89) (end 127 98.806) (width 0.2) (layer "B.Cu") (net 33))
 (segment (start 128.304 79.756) (end 125.222 79.756) (width 0.2) (layer "F.Cu") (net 18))
 (segment (start 129.5 78.56) (end 128.304 79.756) (width 0.2) (layer "F.Cu") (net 18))
 (via (at 125.222 79.756) (size 0.6) (drill 0.3) (layers "F.Cu" "B.Cu") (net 18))
 (segment (start 125.222 79.342) (end 124.45 78.57) (width 0.2) (layer "B.Cu") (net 18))
 (segment (start 125.222 79.756) (end 125.222 79.342) (width 0.2) (layer "B.Cu") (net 18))
 (segment (start 129.5 70.94) (end 128.304 72.136) (width 0.2) (layer "F.Cu") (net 12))
 (segment (start 128.304 72.136) (end 125.222 72.136) (width 0.2) (layer "F.Cu") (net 12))
 (via (at 125.222 72.136) (size 0.6) (drill 0.3) (layers "F.Cu" "B.Cu") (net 12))
 (segment (start 125.222 71.722) (end 124.45 70.95) (width 0.2) (layer "B.Cu") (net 12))
 (segment (start 125.222 72.136) (end 125.222 71.722) (width 0.2) (layer "B.Cu") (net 12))
 (segment (start 129.5 86.18) (end 128.304 87.376) (width 0.2) (layer "F.Cu") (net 24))
 (segment (start 128.304 87.376) (end 125.222 87.376) (width 0.2) (layer "F.Cu") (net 24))
 (via (at 125.222 87.376) (size 0.6) (drill 0.3) (layers "F.Cu" "B.Cu") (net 24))
 (segment (start 125.222 86.962) (end 124.45 86.19) (width 0.2) (layer "B.Cu") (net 24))
 (segment (start 125.222 87.376) (end 125.222 86.962) (width 0.2) (layer "B.Cu") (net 24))
 (segment (start 128.304 102.616) (end 125.222 102.616) (width 0.2) (layer "F.Cu") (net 36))
 (segment (start 129.5 101.42) (end 128.304 102.616) (width 0.2) (layer "F.Cu") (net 36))
 (via (at 125.222 102.616) (size 0.6) (drill 0.3) (layers "F.Cu" "B.Cu") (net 36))
 (segment (start 125.222 102.616) (end 125.222 102.202) (width 0.2) (layer "B.Cu") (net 36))
 (segment (start 125.222 102.202) (end 124.45 101.43) (width 0.2) (layer "B.Cu") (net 36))
 (segment (start 129.5 58.24) (end 128.304 59.436) (width 0.2) (layer "F.Cu") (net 2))
 (segment (start 128.304 59.436) (end 125.222 59.436) (width 0.2) (layer "F.Cu") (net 2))
 (via (at 125.222 59.436) (size 0.6) (drill 0.3) (layers "F.Cu" "B.Cu") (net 2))
 (segment (start 125.222 59.436) (end 125.222 59.022) (width 0.2) (layer "B.Cu") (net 2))
 (segment (start 125.222 59.022) (end 124.45 58.25) (width 0.2) (layer "B.Cu") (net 2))
 (segment (start 128.304 92.456) (end 125.222 92.456) (width 0.2) (layer "F.Cu") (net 28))
 (segment (start 129.5 91.26) (end 128.304 92.456) (width 0.2) (layer "F.Cu") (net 28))
 (via (at 125.222 92.456) (size 0.6) (drill 0.3) (layers "F.Cu" "B.Cu") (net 28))
 (segment (start 125.222 92.456) (end 125.222 92.042) (width 0.2) (layer "B.Cu") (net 28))
 (segment (start 125.222 92.042) (end 124.45 91.27) (width 0.2) (layer "B.Cu") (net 28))
 (segment (start 129.5 65.86) (end 128.304 67.056) (width 0.2) (layer "F.Cu") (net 8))
 (segment (start 128.304 67.056) (end 125.222 67.056) (width 0.2) (layer "F.Cu") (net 8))
 (via (at 125.222 67.056) (size 0.6) (drill 0.3) (layers "F.Cu" "B.Cu") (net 8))
 (segment (start 125.222 67.056) (end 125.222 66.642) (width 0.2) (layer "B.Cu") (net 8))
 (segment (start 125.222 66.642) (end 124.45 65.87) (width 0.2) (layer "B.Cu") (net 8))
 (segment (start 127 91.186) (end 126.492 91.186) (width 0.2) (layer "F.Cu") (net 27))
 (segment (start 126.418 91.26) (end 124.45 91.26) (width 0.2) (layer "F.Cu") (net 27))
 (segment (start 126.492 91.186) (end 126.418 91.26) (width 0.2) (layer "F.Cu") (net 27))
 (via (at 127 91.186) (size 0.6) (drill 0.3) (layers "F.Cu" "B.Cu") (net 27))
 (segment (start 129.5 91.27) (end 127.084 91.27) (width 0.2) (layer "B.Cu") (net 27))
 (segment (start 127.084 91.27) (end 127 91.186) (width 0.2) (layer "B.Cu") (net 27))
 (segment (start 129.5 83.64) (end 128.304 84.836) (width 0.2) (layer "F.Cu") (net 22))
 (segment (start 128.304 84.836) (end 125.222 84.836) (width 0.2) (layer "F.Cu") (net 22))
 (via (at 125.222 84.836) (size 0.6) (drill 0.3) (layers "F.Cu" "B.Cu") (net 22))
 (segment (start 125.222 84.422) (end 124.45 83.65) (width 0.2) (layer "B.Cu") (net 22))
 (segment (start 125.222 84.836) (end 125.222 84.422) (width 0.2) (layer "B.Cu") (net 22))
 (segment (start 127 70.866) (end 124.524 70.866) (width 0.2) (layer "F.Cu") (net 11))
 (segment (start 124.524 70.866) (end 124.45 70.94) (width 0.2) (layer "F.Cu") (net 11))
 (via (at 127 70.866) (size 0.6) (drill 0.3) (layers "F.Cu" "B.Cu") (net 11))
 (segment (start 129.5 70.95) (end 127.084 70.95) (width 0.2) (layer "B.Cu") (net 11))
 (segment (start 127.084 70.95) (end 127 70.866) (width 0.2) (layer "B.Cu") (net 11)))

